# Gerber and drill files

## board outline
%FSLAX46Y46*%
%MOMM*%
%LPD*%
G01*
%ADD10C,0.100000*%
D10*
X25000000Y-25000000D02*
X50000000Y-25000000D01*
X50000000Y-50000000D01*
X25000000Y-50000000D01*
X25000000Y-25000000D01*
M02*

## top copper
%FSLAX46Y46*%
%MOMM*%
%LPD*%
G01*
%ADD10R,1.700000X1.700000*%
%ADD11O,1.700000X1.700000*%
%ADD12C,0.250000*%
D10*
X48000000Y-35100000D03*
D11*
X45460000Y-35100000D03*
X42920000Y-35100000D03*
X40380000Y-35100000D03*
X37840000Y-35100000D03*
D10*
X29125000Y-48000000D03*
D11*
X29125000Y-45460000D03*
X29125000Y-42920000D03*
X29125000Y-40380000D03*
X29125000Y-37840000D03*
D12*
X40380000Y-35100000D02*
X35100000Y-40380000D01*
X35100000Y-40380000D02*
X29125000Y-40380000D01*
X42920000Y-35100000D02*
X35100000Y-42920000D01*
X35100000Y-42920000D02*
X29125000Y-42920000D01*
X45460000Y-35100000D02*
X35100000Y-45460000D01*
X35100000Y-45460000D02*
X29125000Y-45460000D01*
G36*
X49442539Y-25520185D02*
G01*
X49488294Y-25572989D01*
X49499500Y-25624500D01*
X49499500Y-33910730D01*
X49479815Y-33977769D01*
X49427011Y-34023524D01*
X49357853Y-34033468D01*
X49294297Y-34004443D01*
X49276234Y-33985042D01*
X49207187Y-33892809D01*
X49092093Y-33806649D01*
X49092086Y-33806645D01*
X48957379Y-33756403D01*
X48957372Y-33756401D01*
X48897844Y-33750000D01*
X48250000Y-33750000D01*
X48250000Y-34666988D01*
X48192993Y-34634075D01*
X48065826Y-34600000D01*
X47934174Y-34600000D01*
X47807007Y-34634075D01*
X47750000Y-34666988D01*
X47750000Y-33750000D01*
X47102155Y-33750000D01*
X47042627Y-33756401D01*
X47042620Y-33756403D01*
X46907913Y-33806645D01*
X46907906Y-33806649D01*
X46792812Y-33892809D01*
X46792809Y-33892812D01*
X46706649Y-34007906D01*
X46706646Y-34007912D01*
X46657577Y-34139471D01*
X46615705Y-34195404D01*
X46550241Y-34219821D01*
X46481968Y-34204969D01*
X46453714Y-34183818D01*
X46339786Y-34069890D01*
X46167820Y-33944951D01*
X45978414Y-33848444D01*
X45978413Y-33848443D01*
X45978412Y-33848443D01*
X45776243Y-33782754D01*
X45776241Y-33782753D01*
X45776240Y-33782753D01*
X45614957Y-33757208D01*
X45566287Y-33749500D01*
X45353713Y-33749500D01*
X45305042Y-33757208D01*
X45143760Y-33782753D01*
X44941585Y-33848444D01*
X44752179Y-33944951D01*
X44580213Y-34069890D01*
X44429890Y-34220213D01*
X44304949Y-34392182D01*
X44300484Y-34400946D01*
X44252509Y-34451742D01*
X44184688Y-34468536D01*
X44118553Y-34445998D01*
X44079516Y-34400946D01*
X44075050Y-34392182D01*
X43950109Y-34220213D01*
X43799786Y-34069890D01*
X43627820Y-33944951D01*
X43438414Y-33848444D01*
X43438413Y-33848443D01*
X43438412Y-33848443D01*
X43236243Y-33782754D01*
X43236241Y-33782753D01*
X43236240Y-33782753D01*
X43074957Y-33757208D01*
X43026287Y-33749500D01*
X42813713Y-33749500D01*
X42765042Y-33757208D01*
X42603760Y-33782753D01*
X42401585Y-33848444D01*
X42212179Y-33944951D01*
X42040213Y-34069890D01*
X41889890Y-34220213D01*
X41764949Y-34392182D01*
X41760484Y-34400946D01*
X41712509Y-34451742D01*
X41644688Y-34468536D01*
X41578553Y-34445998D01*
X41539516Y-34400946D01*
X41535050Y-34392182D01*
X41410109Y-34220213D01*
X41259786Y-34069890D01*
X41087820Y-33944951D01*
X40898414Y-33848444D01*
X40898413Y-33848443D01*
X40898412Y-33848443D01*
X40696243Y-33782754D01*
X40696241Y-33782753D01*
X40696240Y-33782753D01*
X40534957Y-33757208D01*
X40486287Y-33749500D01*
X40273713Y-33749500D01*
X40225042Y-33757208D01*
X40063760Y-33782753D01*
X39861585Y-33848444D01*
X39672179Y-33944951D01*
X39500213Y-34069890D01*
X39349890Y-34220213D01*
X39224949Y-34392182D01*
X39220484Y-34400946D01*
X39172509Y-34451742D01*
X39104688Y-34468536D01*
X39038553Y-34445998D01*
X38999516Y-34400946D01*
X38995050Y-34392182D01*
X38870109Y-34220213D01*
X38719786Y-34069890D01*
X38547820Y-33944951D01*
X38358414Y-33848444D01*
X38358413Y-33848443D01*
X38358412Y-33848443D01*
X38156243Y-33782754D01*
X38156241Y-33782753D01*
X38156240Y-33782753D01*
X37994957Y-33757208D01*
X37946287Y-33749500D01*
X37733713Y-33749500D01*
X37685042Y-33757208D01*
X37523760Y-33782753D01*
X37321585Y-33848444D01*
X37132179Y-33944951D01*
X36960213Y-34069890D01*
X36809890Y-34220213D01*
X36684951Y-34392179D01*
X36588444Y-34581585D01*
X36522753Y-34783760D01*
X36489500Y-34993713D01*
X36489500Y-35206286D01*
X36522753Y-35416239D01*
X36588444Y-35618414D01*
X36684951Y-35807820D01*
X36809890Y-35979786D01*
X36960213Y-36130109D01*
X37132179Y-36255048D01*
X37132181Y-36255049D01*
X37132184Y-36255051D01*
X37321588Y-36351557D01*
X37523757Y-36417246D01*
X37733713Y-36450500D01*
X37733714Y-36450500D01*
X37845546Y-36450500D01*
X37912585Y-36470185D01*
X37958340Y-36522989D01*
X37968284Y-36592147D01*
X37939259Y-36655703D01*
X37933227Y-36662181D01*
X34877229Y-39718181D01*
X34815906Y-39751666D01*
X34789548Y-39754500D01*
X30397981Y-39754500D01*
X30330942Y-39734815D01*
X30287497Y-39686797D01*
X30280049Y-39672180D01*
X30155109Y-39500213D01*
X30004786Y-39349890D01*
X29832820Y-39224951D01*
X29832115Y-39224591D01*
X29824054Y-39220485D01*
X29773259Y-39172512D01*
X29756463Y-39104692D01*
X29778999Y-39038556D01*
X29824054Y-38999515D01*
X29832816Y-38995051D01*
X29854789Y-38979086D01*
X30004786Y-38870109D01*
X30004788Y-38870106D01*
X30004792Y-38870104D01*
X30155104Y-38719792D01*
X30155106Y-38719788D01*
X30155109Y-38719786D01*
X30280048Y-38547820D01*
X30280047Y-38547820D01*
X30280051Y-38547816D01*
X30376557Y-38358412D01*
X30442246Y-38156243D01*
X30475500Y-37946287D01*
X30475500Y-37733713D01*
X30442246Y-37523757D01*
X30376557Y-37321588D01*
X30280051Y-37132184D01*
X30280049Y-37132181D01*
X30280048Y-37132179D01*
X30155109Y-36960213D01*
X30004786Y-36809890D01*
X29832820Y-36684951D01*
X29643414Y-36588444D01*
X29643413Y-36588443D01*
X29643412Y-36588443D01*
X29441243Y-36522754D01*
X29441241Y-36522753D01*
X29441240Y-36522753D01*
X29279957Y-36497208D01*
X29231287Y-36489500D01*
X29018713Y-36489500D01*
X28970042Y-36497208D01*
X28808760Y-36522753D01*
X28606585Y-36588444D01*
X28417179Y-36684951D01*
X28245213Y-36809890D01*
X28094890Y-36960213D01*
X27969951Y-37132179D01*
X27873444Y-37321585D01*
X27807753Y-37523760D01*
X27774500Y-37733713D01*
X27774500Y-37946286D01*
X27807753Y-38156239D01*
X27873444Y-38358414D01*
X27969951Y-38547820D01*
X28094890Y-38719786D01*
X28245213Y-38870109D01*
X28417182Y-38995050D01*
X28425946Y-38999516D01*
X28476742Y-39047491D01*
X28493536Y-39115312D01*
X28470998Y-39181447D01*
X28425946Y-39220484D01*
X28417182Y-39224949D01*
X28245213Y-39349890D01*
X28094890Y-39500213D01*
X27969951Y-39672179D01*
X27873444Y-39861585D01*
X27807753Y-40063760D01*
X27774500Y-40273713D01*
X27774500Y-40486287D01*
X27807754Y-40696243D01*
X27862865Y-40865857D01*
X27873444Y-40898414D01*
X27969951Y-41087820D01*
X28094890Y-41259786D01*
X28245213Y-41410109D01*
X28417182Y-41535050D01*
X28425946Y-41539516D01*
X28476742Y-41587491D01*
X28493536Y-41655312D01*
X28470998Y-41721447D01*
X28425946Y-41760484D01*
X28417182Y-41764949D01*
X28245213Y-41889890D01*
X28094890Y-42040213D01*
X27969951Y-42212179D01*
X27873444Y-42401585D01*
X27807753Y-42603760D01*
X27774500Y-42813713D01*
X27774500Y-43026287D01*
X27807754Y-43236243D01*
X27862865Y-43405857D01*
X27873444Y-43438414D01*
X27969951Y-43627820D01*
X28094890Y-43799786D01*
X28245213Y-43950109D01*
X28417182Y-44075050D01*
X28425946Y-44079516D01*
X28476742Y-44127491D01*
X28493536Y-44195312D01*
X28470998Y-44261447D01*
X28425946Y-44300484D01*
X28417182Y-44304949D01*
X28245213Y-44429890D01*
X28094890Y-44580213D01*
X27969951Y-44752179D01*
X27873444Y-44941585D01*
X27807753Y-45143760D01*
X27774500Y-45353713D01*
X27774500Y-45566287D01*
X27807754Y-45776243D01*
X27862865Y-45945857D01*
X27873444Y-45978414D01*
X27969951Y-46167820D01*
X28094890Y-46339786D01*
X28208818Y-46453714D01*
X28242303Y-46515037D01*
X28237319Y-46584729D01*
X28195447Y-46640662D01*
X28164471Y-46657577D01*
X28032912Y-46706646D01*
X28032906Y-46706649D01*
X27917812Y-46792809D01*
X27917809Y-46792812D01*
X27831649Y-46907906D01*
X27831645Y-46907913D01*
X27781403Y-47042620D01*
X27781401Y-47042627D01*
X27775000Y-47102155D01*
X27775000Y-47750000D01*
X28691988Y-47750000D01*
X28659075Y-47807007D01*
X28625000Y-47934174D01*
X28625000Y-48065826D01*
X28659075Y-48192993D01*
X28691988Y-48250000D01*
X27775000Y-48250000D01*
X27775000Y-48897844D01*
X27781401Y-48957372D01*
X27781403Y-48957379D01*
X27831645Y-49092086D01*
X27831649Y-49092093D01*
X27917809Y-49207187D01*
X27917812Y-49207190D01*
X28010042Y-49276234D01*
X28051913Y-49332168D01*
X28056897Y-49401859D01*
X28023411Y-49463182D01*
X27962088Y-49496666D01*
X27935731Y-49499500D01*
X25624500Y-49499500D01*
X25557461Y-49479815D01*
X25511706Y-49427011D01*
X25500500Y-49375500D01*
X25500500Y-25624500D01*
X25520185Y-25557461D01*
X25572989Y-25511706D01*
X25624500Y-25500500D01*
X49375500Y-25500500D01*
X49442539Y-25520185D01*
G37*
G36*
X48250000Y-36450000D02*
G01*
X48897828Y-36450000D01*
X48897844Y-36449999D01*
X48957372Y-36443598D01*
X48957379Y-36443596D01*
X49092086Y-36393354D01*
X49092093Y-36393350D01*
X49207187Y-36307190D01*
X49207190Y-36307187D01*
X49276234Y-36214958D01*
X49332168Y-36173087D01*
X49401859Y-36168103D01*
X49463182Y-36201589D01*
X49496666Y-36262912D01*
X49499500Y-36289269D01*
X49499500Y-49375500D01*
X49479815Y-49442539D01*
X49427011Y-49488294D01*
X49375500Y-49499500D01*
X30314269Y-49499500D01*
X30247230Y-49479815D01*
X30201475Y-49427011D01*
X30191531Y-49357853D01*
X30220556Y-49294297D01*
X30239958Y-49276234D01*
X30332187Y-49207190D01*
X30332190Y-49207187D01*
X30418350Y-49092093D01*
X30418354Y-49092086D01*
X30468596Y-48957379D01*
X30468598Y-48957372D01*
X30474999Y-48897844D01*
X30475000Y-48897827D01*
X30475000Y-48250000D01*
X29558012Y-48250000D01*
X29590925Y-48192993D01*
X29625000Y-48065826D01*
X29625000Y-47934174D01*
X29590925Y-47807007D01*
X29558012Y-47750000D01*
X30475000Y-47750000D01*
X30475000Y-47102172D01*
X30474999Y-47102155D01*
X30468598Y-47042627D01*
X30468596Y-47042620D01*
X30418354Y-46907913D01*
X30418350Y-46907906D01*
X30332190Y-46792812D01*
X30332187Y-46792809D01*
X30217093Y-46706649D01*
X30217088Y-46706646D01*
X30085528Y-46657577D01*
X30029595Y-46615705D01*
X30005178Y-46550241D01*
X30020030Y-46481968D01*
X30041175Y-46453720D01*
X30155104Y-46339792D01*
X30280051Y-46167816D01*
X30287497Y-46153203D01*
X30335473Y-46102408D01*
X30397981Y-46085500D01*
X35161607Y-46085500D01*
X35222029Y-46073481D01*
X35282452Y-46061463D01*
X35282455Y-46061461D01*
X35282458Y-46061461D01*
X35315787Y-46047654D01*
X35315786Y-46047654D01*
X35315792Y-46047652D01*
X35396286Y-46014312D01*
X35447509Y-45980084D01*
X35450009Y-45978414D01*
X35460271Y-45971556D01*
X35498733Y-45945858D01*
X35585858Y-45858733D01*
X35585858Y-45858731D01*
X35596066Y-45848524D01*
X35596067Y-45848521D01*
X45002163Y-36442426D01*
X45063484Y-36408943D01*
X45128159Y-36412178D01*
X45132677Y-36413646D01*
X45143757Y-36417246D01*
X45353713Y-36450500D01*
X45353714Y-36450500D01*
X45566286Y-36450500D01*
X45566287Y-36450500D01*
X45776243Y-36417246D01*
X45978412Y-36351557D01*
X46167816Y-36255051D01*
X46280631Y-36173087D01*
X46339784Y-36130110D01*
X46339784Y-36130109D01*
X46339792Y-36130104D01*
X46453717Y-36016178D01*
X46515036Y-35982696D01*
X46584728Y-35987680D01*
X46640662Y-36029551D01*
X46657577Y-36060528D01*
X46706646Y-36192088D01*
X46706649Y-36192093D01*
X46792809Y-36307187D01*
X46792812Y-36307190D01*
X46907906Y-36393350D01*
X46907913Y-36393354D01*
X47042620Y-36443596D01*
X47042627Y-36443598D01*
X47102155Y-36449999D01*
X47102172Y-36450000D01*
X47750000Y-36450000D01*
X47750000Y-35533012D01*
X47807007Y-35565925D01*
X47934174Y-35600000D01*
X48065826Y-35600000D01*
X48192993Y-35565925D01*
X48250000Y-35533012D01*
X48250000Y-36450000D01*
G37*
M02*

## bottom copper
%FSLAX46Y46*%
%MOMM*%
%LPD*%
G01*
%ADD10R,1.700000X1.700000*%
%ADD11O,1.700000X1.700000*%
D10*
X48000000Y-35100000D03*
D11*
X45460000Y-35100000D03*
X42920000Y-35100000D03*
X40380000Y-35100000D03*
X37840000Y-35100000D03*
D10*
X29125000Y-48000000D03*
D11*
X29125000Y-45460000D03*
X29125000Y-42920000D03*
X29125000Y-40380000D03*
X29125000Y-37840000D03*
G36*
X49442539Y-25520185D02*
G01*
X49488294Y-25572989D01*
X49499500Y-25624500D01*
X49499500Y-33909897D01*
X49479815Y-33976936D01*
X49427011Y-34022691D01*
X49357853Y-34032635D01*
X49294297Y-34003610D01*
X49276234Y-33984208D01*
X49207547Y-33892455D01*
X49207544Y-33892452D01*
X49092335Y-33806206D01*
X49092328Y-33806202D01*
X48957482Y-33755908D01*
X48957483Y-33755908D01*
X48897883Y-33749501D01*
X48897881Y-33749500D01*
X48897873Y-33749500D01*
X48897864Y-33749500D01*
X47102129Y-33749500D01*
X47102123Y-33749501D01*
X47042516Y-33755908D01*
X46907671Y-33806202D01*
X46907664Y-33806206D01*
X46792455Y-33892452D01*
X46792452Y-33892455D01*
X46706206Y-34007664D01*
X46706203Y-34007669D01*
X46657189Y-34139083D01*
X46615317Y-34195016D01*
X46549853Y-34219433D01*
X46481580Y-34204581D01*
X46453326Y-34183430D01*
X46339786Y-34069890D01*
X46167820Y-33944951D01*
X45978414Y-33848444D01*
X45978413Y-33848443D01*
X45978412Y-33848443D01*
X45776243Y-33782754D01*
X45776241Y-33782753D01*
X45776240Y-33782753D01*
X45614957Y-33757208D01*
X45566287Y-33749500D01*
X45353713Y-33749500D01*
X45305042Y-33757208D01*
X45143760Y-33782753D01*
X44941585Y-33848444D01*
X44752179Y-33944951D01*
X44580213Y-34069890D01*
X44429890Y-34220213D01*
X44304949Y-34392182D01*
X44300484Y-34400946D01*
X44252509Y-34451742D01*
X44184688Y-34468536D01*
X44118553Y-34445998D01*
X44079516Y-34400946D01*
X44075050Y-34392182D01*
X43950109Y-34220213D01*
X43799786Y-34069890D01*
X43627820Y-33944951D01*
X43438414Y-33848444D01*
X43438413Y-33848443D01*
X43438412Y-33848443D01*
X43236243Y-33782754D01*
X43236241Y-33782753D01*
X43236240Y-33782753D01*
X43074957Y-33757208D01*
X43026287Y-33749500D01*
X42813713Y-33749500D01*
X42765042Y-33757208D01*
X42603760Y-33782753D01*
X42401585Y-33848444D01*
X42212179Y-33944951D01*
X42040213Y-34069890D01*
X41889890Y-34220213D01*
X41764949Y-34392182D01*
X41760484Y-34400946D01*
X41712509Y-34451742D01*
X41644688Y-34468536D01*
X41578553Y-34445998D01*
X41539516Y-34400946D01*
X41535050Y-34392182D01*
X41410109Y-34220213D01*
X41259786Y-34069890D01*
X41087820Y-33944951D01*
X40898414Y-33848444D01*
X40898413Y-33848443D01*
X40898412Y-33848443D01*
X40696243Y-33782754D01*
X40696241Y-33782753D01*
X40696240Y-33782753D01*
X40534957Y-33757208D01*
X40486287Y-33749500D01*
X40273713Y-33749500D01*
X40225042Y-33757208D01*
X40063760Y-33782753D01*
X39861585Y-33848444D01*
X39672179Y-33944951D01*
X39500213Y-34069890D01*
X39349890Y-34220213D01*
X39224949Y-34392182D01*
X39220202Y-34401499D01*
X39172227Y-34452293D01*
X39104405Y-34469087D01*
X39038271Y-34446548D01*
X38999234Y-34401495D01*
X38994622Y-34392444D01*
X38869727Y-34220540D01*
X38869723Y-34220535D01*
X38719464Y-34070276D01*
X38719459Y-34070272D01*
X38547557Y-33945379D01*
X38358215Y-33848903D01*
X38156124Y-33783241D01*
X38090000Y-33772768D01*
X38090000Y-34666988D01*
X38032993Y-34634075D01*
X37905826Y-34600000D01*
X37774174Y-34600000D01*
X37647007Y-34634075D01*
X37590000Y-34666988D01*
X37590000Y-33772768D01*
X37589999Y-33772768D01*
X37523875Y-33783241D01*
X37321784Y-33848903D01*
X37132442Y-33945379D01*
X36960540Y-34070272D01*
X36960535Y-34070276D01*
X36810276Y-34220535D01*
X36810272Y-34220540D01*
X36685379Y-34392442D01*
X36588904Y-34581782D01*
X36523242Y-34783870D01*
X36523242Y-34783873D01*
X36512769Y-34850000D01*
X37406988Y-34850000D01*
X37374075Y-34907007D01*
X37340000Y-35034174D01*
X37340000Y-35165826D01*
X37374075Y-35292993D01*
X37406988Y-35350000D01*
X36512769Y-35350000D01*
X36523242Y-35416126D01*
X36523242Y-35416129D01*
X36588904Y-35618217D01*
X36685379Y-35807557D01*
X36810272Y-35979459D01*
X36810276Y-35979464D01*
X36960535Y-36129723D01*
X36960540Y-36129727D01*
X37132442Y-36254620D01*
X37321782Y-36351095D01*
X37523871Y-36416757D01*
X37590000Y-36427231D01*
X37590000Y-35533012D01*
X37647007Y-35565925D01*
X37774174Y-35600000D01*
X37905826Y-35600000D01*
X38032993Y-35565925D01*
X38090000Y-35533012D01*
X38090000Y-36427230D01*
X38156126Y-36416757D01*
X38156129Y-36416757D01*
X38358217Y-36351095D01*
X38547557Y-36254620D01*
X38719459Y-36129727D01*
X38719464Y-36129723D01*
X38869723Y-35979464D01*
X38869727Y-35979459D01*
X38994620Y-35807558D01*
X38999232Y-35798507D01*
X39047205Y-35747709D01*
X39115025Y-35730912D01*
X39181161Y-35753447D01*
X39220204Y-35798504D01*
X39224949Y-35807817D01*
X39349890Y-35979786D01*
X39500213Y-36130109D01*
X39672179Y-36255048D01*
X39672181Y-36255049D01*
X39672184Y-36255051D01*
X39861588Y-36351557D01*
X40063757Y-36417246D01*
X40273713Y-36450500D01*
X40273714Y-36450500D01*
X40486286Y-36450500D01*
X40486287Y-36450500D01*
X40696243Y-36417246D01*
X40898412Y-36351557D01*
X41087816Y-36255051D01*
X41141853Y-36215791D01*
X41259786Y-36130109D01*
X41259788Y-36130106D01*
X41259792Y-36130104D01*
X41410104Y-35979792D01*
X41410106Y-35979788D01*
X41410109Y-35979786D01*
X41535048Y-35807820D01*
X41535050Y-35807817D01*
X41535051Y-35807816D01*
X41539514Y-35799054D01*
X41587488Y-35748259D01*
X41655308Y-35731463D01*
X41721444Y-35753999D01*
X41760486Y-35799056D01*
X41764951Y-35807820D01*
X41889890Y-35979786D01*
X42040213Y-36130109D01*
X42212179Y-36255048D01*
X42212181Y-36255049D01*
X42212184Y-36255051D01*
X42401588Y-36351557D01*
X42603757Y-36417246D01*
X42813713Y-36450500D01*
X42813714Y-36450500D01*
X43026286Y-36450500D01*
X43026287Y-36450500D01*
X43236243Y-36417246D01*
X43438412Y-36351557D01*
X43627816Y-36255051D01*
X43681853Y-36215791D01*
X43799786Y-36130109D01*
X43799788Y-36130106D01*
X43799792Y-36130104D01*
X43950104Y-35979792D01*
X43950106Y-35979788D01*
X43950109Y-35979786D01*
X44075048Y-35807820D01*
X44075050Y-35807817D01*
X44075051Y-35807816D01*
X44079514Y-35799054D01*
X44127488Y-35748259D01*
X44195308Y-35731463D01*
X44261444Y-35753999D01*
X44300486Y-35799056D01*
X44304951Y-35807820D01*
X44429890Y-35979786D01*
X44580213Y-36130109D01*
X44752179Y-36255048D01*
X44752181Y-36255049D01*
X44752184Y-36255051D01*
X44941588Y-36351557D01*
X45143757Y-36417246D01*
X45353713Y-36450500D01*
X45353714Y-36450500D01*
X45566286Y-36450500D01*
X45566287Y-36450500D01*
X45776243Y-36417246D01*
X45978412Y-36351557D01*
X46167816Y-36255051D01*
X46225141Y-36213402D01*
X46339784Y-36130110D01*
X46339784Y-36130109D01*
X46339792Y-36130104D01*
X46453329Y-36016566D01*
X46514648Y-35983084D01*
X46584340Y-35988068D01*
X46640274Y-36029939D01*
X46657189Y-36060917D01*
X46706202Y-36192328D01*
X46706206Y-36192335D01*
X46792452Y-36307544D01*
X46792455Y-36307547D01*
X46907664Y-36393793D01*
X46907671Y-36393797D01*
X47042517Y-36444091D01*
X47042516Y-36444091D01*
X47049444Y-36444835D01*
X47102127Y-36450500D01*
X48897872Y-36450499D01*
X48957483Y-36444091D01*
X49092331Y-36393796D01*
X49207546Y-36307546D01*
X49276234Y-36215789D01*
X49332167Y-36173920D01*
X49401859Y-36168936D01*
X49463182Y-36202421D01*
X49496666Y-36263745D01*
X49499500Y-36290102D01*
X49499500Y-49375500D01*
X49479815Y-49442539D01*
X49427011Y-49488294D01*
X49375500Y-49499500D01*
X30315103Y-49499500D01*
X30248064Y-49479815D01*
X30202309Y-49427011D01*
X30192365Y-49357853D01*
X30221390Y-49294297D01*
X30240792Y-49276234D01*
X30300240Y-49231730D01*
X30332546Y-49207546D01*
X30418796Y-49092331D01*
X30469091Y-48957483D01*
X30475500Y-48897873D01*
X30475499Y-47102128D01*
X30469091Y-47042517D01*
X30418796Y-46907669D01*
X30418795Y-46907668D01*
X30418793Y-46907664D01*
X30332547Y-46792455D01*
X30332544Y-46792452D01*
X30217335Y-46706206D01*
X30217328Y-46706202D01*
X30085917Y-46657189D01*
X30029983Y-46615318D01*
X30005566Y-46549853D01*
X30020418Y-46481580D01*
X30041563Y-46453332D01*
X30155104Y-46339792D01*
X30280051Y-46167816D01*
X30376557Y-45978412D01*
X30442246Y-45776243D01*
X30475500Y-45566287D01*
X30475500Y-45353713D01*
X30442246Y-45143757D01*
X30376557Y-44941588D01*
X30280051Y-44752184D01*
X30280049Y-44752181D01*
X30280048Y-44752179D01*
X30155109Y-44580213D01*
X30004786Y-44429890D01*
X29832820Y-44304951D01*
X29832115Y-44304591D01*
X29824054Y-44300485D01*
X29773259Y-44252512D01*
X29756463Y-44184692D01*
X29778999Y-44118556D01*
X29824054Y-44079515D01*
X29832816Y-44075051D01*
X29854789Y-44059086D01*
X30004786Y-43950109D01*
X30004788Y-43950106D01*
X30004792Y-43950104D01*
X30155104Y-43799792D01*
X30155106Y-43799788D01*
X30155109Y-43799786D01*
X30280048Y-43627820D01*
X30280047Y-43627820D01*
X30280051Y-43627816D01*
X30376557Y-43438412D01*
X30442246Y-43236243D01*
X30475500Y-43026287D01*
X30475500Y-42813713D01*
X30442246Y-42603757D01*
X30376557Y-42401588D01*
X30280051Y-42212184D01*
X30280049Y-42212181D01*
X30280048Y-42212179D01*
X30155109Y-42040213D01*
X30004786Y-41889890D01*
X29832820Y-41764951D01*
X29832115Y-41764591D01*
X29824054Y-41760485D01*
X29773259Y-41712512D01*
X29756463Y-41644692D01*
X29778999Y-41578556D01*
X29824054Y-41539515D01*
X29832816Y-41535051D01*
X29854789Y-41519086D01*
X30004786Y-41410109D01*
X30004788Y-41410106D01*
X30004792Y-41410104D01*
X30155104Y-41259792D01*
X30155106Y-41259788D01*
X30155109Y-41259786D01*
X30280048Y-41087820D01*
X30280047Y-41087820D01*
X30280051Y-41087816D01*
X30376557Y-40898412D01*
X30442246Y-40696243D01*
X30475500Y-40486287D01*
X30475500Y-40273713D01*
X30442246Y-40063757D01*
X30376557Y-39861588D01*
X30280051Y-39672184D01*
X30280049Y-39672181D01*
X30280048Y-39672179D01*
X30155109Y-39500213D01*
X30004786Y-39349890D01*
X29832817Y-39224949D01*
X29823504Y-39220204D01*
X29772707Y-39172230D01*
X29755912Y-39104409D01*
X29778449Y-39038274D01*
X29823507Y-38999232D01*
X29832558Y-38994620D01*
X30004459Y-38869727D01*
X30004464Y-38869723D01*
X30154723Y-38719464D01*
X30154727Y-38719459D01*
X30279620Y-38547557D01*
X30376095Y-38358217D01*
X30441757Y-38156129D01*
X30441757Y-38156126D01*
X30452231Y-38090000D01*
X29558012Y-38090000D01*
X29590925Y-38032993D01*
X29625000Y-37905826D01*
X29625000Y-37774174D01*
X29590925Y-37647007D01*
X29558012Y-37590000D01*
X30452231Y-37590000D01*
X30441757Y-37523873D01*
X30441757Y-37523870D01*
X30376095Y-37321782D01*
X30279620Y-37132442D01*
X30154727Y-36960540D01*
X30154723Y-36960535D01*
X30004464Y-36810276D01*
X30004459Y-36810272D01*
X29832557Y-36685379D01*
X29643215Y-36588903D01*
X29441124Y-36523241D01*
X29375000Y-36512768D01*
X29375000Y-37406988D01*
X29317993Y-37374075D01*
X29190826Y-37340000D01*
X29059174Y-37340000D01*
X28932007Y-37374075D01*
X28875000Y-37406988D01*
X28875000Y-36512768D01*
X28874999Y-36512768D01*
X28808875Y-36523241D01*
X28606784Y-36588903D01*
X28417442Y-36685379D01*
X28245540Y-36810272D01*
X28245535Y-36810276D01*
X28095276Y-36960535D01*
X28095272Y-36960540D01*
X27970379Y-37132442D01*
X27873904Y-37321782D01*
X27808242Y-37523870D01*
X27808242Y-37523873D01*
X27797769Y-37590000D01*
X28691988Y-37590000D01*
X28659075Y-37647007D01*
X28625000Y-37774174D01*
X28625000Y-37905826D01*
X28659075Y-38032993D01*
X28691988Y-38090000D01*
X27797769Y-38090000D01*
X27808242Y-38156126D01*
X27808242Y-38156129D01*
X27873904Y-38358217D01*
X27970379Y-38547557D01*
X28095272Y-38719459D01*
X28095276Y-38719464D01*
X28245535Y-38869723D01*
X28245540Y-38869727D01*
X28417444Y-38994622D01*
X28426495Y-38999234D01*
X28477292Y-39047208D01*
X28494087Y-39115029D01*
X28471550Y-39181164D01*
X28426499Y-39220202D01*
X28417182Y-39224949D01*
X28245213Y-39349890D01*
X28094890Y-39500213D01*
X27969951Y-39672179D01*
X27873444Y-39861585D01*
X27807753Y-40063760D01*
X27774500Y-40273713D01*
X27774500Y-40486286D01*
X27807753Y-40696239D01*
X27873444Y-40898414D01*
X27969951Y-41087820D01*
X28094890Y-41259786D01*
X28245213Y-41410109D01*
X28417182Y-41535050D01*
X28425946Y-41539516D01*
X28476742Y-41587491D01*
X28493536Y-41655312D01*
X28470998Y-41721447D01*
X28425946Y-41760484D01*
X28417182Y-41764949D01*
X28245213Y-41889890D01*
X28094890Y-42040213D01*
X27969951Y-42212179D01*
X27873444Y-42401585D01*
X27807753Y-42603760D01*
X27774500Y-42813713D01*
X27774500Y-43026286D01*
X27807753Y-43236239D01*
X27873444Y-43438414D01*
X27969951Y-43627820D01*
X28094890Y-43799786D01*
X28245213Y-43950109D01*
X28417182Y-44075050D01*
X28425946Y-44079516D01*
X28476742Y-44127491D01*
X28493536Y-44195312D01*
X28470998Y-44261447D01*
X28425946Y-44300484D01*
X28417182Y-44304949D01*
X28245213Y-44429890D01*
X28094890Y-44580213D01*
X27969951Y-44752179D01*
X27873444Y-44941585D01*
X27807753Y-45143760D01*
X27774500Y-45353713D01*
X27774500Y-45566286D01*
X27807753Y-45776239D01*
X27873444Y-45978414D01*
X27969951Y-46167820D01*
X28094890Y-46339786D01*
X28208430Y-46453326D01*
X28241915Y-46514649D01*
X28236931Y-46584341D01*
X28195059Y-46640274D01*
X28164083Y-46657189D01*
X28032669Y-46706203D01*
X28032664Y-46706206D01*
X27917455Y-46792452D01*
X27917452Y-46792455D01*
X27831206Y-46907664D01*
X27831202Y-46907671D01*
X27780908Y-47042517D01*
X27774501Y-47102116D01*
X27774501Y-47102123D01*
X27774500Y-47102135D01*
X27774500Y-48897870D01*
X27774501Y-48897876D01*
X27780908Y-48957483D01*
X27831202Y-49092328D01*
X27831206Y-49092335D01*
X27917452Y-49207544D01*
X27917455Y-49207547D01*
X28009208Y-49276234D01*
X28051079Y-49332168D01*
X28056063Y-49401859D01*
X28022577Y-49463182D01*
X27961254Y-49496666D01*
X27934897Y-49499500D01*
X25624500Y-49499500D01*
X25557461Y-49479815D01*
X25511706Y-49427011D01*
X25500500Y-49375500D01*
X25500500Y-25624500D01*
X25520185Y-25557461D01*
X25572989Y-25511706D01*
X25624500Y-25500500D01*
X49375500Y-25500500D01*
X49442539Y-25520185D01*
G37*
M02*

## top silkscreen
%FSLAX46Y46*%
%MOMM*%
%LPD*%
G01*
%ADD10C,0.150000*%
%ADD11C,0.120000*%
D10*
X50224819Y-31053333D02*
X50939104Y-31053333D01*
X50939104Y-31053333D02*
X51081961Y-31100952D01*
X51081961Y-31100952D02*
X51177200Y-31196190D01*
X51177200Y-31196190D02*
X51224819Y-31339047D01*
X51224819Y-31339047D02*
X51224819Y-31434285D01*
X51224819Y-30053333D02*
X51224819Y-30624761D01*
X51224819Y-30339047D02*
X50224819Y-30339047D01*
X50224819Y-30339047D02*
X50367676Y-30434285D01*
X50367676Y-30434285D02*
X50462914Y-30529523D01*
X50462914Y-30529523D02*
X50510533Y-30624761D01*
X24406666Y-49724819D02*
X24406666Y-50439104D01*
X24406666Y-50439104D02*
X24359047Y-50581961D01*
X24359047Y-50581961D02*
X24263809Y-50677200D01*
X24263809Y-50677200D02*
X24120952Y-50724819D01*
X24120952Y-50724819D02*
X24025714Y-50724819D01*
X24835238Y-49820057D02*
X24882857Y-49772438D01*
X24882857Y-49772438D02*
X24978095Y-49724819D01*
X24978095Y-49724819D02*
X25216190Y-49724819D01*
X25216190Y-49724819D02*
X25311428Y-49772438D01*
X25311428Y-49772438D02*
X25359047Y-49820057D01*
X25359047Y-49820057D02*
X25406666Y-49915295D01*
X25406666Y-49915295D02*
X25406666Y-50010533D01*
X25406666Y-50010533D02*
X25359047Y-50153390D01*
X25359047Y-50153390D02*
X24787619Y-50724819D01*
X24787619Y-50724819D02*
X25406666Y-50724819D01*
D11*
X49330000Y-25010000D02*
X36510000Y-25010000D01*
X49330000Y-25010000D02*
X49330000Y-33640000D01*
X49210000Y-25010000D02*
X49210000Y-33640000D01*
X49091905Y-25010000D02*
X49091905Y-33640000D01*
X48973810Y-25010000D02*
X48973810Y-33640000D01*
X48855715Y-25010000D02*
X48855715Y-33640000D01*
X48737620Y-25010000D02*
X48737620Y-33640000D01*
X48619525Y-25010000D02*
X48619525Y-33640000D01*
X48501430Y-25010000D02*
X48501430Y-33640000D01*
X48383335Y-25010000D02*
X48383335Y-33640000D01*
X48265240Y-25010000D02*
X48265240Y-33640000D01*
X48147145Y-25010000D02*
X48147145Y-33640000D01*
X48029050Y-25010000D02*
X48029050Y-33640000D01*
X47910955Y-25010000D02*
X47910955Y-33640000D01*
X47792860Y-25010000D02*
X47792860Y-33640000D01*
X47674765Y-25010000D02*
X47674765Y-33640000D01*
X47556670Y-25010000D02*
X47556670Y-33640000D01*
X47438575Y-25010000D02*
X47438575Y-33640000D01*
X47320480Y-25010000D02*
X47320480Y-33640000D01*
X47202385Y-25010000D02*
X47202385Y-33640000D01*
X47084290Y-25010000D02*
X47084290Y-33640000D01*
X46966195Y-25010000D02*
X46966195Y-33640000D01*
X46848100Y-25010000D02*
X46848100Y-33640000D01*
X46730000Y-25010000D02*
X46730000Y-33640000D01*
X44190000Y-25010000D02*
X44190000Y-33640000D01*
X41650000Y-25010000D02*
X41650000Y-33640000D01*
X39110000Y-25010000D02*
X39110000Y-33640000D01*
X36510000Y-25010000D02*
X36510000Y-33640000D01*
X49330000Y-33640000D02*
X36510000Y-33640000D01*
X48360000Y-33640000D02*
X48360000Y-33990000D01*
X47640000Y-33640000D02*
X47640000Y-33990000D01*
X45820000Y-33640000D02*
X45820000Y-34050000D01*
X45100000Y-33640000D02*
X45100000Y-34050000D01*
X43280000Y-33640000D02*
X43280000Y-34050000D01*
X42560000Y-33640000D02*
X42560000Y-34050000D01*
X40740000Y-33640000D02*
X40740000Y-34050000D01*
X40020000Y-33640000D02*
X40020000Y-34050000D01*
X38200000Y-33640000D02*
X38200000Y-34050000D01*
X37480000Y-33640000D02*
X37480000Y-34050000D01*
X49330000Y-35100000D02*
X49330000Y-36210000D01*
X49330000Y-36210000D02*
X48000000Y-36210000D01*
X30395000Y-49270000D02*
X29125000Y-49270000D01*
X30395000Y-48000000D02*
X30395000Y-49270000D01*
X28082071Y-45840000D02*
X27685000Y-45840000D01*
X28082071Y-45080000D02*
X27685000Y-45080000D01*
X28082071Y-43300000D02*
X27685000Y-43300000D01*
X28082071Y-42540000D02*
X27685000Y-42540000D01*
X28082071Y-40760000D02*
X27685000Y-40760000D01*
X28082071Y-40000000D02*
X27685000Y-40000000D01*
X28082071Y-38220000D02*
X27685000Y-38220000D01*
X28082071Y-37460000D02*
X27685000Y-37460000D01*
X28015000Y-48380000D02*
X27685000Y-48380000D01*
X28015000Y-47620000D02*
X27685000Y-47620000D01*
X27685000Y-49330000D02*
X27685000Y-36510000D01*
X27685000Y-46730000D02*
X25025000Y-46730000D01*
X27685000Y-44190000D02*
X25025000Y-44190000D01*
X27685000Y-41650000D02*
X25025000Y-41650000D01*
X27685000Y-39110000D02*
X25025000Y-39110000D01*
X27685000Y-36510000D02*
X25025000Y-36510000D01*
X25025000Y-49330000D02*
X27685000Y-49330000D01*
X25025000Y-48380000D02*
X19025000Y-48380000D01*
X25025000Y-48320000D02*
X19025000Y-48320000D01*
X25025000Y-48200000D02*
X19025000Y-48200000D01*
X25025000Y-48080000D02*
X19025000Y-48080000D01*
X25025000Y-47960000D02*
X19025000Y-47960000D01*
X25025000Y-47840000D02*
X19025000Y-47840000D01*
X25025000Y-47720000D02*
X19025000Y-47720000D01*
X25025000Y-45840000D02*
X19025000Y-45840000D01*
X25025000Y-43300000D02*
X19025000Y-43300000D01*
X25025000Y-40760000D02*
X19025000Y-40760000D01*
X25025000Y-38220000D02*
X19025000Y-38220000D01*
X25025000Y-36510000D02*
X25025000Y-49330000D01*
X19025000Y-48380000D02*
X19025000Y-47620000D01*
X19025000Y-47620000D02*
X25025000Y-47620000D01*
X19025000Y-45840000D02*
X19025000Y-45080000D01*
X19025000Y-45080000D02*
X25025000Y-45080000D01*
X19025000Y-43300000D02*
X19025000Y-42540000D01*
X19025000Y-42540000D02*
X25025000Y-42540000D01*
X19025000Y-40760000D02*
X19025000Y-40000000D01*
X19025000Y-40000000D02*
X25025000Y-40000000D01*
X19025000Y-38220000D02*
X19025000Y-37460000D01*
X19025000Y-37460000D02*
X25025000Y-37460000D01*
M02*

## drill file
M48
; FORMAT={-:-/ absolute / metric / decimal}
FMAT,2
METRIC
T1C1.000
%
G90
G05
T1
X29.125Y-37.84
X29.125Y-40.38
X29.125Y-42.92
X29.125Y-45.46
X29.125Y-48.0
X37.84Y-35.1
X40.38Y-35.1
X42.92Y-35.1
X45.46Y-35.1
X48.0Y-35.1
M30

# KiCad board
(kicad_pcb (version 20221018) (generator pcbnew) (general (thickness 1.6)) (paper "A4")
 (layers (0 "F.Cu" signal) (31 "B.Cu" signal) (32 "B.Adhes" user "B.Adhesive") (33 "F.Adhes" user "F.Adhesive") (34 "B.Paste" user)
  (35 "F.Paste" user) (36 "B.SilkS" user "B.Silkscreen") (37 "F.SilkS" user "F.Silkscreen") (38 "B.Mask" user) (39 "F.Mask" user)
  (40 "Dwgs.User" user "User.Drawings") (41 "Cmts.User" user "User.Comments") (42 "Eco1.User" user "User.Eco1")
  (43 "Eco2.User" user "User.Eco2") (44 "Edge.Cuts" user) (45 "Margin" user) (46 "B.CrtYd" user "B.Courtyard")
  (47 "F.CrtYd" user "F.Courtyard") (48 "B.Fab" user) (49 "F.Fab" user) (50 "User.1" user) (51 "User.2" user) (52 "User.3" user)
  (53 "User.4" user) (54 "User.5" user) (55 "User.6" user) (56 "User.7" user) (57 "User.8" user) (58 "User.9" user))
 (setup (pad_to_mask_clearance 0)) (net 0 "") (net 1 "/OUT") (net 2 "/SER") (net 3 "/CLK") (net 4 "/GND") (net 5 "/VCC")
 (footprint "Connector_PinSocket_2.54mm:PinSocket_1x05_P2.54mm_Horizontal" (layer "F.Cu") (at 48 35.1 -90)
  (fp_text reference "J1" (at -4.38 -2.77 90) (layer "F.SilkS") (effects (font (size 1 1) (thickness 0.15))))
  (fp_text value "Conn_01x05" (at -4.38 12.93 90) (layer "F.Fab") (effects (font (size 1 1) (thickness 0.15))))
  (fp_line (start -10.09 -1.33) (end -10.09 11.49) (stroke (width 0.12) (type solid)) (layer "F.SilkS"))
  (fp_line (start -10.09 -1.33) (end -1.46 -1.33) (stroke (width 0.12) (type solid)) (layer "F.SilkS"))
  (fp_line (start -10.09 -1.21) (end -1.46 -1.21) (stroke (width 0.12) (type solid)) (layer "F.SilkS"))
  (fp_line (start -10.09 -1.091905) (end -1.46 -1.091905) (stroke (width 0.12) (type solid)) (layer "F.SilkS"))
  (fp_line (start -10.09 -0.97381) (end -1.46 -0.97381) (stroke (width 0.12) (type solid)) (layer "F.SilkS"))
  (fp_line (start -10.09 -0.855715) (end -1.46 -0.855715) (stroke (width 0.12) (type solid)) (layer "F.SilkS"))
  (fp_line (start -10.09 -0.73762) (end -1.46 -0.73762) (stroke (width 0.12) (type solid)) (layer "F.SilkS"))
  (fp_line (start -10.09 -0.619525) (end -1.46 -0.619525) (stroke (width 0.12) (type solid)) (layer "F.SilkS"))
  (fp_line (start -10.09 -0.50143) (end -1.46 -0.50143) (stroke (width 0.12) (type solid)) (layer "F.SilkS"))
  (fp_line (start -10.09 -0.383335) (end -1.46 -0.383335) (stroke (width 0.12) (type solid)) (layer "F.SilkS"))
  (fp_line (start -10.09 -0.26524) (end -1.46 -0.26524) (stroke (width 0.12) (type solid)) (layer "F.SilkS"))
  (fp_line (start -10.09 -0.147145) (end -1.46 -0.147145) (stroke (width 0.12) (type solid)) (layer "F.SilkS"))
  (fp_line (start -10.09 -0.02905) (end -1.46 -0.02905) (stroke (width 0.12) (type solid)) (layer "F.SilkS"))
  (fp_line (start -10.09 0.089045) (end -1.46 0.089045) (stroke (width 0.12) (type solid)) (layer "F.SilkS"))
  (fp_line (start -10.09 0.20714) (end -1.46 0.20714) (stroke (width 0.12) (type solid)) (layer "F.SilkS"))
  (fp_line (start -10.09 0.325235) (end -1.46 0.325235) (stroke (width 0.12) (type solid)) (layer "F.SilkS"))
  (fp_line (start -10.09 0.44333) (end -1.46 0.44333) (stroke (width 0.12) (type solid)) (layer "F.SilkS"))
  (fp_line (start -10.09 0.561425) (end -1.46 0.561425) (stroke (width 0.12) (type solid)) (layer "F.SilkS"))
  (fp_line (start -10.09 0.67952) (end -1.46 0.67952) (stroke (width 0.12) (type solid)) (layer "F.SilkS"))
  (fp_line (start -10.09 0.797615) (end -1.46 0.797615) (stroke (width 0.12) (type solid)) (layer "F.SilkS"))
  (fp_line (start -10.09 0.91571) (end -1.46 0.91571) (stroke (width 0.12) (type solid)) (layer "F.SilkS"))
  (fp_line (start -10.09 1.033805) (end -1.46 1.033805) (stroke (width 0.12) (type solid)) (layer "F.SilkS"))
  (fp_line (start -10.09 1.1519) (end -1.46 1.1519) (stroke (width 0.12) (type solid)) (layer "F.SilkS"))
  (fp_line (start -10.09 1.27) (end -1.46 1.27) (stroke (width 0.12) (type solid)) (layer "F.SilkS"))
  (fp_line (start -10.09 3.81) (end -1.46 3.81) (stroke (width 0.12) (type solid)) (layer "F.SilkS"))
  (fp_line (start -10.09 6.35) (end -1.46 6.35) (stroke (width 0.12) (type solid)) (layer "F.SilkS"))
  (fp_line (start -10.09 8.89) (end -1.46 8.89) (stroke (width 0.12) (type solid)) (layer "F.SilkS"))
  (fp_line (start -10.09 11.49) (end -1.46 11.49) (stroke (width 0.12) (type solid)) (layer "F.SilkS"))
  (fp_line (start -1.46 -1.33) (end -1.46 11.49) (stroke (width 0.12) (type solid)) (layer "F.SilkS"))
  (fp_line (start -1.46 -0.36) (end -1.11 -0.36) (stroke (width 0.12) (type solid)) (layer "F.SilkS"))
  (fp_line (start -1.46 0.36) (end -1.11 0.36) (stroke (width 0.12) (type solid)) (layer "F.SilkS"))
  (fp_line (start -1.46 2.18) (end -1.05 2.18) (stroke (width 0.12) (type solid)) (layer "F.SilkS"))
  (fp_line (start -1.46 2.9) (end -1.05 2.9) (stroke (width 0.12) (type solid)) (layer "F.SilkS"))
  (fp_line (start -1.46 4.72) (end -1.05 4.72) (stroke (width 0.12) (type solid)) (layer "F.SilkS"))
  (fp_line (start -1.46 5.44) (end -1.05 5.44) (stroke (width 0.12) (type solid)) (layer "F.SilkS"))
  (fp_line (start -1.46 7.26) (end -1.05 7.26) (stroke (width 0.12) (type solid)) (layer "F.SilkS"))
  (fp_line (start -1.46 7.98) (end -1.05 7.98) (stroke (width 0.12) (type solid)) (layer "F.SilkS"))
  (fp_line (start -1.46 9.8) (end -1.05 9.8) (stroke (width 0.12) (type solid)) (layer "F.SilkS"))
  (fp_line (start -1.46 10.52) (end -1.05 10.52) (stroke (width 0.12) (type solid)) (layer "F.SilkS"))
  (fp_line (start 0 -1.33) (end 1.11 -1.33) (stroke (width 0.12) (type solid)) (layer "F.SilkS"))
  (fp_line (start 1.11 -1.33) (end 1.11 0) (stroke (width 0.12) (type solid)) (layer "F.SilkS"))
  (pad "1" thru_hole rect (at 0 0 270) (size 1.7 1.7) (drill 1) (layers "*.Cu" "*.Mask") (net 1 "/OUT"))
  (pad "2" thru_hole oval (at 0 2.54 270) (size 1.7 1.7) (drill 1) (layers "*.Cu" "*.Mask") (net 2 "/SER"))
  (pad "3" thru_hole oval (at 0 5.08 270) (size 1.7 1.7) (drill 1) (layers "*.Cu" "*.Mask") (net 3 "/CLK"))
  (pad "4" thru_hole oval (at 0 7.62 270) (size 1.7 1.7) (drill 1) (layers "*.Cu" "*.Mask") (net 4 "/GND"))
  (pad "5" thru_hole oval (at 0 10.16 270) (size 1.7 1.7) (drill 1) (layers "*.Cu" "*.Mask") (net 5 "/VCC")))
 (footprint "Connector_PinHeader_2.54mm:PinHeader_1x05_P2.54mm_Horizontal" (layer "F.Cu") (at 29.125 48 180)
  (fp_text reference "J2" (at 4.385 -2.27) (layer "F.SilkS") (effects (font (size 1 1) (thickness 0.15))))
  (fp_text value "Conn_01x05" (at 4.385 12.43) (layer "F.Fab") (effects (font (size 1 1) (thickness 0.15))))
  (fp_line (start -1.27 -1.27) (end 0 -1.27) (stroke (width 0.12) (type solid)) (layer "F.SilkS"))
  (fp_line (start -1.27 0) (end -1.27 -1.27) (stroke (width 0.12) (type solid)) (layer "F.SilkS"))
  (fp_line (start 1.042929 2.16) (end 1.44 2.16) (stroke (width 0.12) (type solid)) (layer "F.SilkS"))
  (fp_line (start 1.042929 2.92) (end 1.44 2.92) (stroke (width 0.12) (type solid)) (layer "F.SilkS"))
  (fp_line (start 1.042929 4.7) (end 1.44 4.7) (stroke (width 0.12) (type solid)) (layer "F.SilkS"))
  (fp_line (start 1.042929 5.46) (end 1.44 5.46) (stroke (width 0.12) (type solid)) (layer "F.SilkS"))
  (fp_line (start 1.042929 7.24) (end 1.44 7.24) (stroke (width 0.12) (type solid)) (layer "F.SilkS"))
  (fp_line (start 1.042929 8) (end 1.44 8) (stroke (width 0.12) (type solid)) (layer "F.SilkS"))
  (fp_line (start 1.042929 9.78) (end 1.44 9.78) (stroke (width 0.12) (type solid)) (layer "F.SilkS"))
  (fp_line (start 1.042929 10.54) (end 1.44 10.54) (stroke (width 0.12) (type solid)) (layer "F.SilkS"))
  (fp_line (start 1.11 -0.38) (end 1.44 -0.38) (stroke (width 0.12) (type solid)) (layer "F.SilkS"))
  (fp_line (start 1.11 0.38) (end 1.44 0.38) (stroke (width 0.12) (type solid)) (layer "F.SilkS"))
  (fp_line (start 1.44 -1.33) (end 1.44 11.49) (stroke (width 0.12) (type solid)) (layer "F.SilkS"))
  (fp_line (start 1.44 1.27) (end 4.1 1.27) (stroke (width 0.12) (type solid)) (layer "F.SilkS"))
  (fp_line (start 1.44 3.81) (end 4.1 3.81) (stroke (width 0.12) (type solid)) (layer "F.SilkS"))
  (fp_line (start 1.44 6.35) (end 4.1 6.35) (stroke (width 0.12) (type solid)) (layer "F.SilkS"))
  (fp_line (start 1.44 8.89) (end 4.1 8.89) (stroke (width 0.12) (type solid)) (layer "F.SilkS"))
  (fp_line (start 1.44 11.49) (end 4.1 11.49) (stroke (width 0.12) (type solid)) (layer "F.SilkS"))
  (fp_line (start 4.1 -1.33) (end 1.44 -1.33) (stroke (width 0.12) (type solid)) (layer "F.SilkS"))
  (fp_line (start 4.1 -0.38) (end 10.1 -0.38) (stroke (width 0.12) (type solid)) (layer "F.SilkS"))
  (fp_line (start 4.1 -0.32) (end 10.1 -0.32) (stroke (width 0.12) (type solid)) (layer "F.SilkS"))
  (fp_line (start 4.1 -0.2) (end 10.1 -0.2) (stroke (width 0.12) (type solid)) (layer "F.SilkS"))
  (fp_line (start 4.1 -0.08) (end 10.1 -0.08) (stroke (width 0.12) (type solid)) (layer "F.SilkS"))
  (fp_line (start 4.1 0.04) (end 10.1 0.04) (stroke (width 0.12) (type solid)) (layer "F.SilkS"))
  (fp_line (start 4.1 0.16) (end 10.1 0.16) (stroke (width 0.12) (type solid)) (layer "F.SilkS"))
  (fp_line (start 4.1 0.28) (end 10.1 0.28) (stroke (width 0.12) (type solid)) (layer "F.SilkS"))
  (fp_line (start 4.1 2.16) (end 10.1 2.16) (stroke (width 0.12) (type solid)) (layer "F.SilkS"))
  (fp_line (start 4.1 4.7) (end 10.1 4.7) (stroke (width 0.12) (type solid)) (layer "F.SilkS"))
  (fp_line (start 4.1 7.24) (end 10.1 7.24) (stroke (width 0.12) (type solid)) (layer "F.SilkS"))
  (fp_line (start 4.1 9.78) (end 10.1 9.78) (stroke (width 0.12) (type solid)) (layer "F.SilkS"))
  (fp_line (start 4.1 11.49) (end 4.1 -1.33) (stroke (width 0.12) (type solid)) (layer "F.SilkS"))
  (fp_line (start 10.1 -0.38) (end 10.1 0.38) (stroke (width 0.12) (type solid)) (layer "F.SilkS"))
  (fp_line (start 10.1 0.38) (end 4.1 0.38) (stroke (width 0.12) (type solid)) (layer "F.SilkS"))
  (fp_line (start 10.1 2.16) (end 10.1 2.92) (stroke (width 0.12) (type solid)) (layer "F.SilkS"))
  (fp_line (start 10.1 2.92) (end 4.1 2.92) (stroke (width 0.12) (type solid)) (layer "F.SilkS"))
  (fp_line (start 10.1 4.7) (end 10.1 5.46) (stroke (width 0.12) (type solid)) (layer "F.SilkS"))
  (fp_line (start 10.1 5.46) (end 4.1 5.46) (stroke (width 0.12) (type solid)) (layer "F.SilkS"))
  (fp_line (start 10.1 7.24) (end 10.1 8) (stroke (width 0.12) (type solid)) (layer "F.SilkS"))
  (fp_line (start 10.1 8) (end 4.1 8) (stroke (width 0.12) (type solid)) (layer "F.SilkS"))
  (fp_line (start 10.1 9.78) (end 10.1 10.54) (stroke (width 0.12) (type solid)) (layer "F.SilkS"))
  (fp_line (start 10.1 10.54) (end 4.1 10.54) (stroke (width 0.12) (type solid)) (layer "F.SilkS"))
  (pad "1" thru_hole rect (at 0 0 180) (size 1.7 1.7) (drill 1) (layers "*.Cu" "*.Mask") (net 1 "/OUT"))
  (pad "2" thru_hole oval (at 0 2.54 180) (size 1.7 1.7) (drill 1) (layers "*.Cu" "*.Mask") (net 2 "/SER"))
  (pad "3" thru_hole oval (at 0 5.08 180) (size 1.7 1.7) (drill 1) (layers "*.Cu" "*.Mask") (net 3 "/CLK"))
  (pad "4" thru_hole oval (at 0 7.62 180) (size 1.7 1.7) (drill 1) (layers "*.Cu" "*.Mask") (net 4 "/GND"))
  (pad "5" thru_hole oval (at 0 10.16 180) (size 1.7 1.7) (drill 1) (layers "*.Cu" "*.Mask") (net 5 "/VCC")))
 (gr_rect (start 25 25) (end 50 50) (stroke (width 0.1) (type default)) (fill none) (layer "Edge.Cuts"))
 (segment (start 40.38 35.1) (end 35.1 40.38) (width 0.25) (layer "F.Cu") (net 4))
 (segment (start 35.1 40.38) (end 29.125 40.38) (width 0.25) (layer "F.Cu") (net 4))
 (segment (start 42.92 35.1) (end 35.1 42.92) (width 0.25) (layer "F.Cu") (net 3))
 (segment (start 35.1 42.92) (end 29.125 42.92) (width 0.25) (layer "F.Cu") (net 3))
 (segment (start 45.46 35.1) (end 35.1 45.46) (width 0.25) (layer "F.Cu") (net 2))
 (segment (start 35.1 45.46) (end 29.125 45.46) (width 0.25) (layer "F.Cu") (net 2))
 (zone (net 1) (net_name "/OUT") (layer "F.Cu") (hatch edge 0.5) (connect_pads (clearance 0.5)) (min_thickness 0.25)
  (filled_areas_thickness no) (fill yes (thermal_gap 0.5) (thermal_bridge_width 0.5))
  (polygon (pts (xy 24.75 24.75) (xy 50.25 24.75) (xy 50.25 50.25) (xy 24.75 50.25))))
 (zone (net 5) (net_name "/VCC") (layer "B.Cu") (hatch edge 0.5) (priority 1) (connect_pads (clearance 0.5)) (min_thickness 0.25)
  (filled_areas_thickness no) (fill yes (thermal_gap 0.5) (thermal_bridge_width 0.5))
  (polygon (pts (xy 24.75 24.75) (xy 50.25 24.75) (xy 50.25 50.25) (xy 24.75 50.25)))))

